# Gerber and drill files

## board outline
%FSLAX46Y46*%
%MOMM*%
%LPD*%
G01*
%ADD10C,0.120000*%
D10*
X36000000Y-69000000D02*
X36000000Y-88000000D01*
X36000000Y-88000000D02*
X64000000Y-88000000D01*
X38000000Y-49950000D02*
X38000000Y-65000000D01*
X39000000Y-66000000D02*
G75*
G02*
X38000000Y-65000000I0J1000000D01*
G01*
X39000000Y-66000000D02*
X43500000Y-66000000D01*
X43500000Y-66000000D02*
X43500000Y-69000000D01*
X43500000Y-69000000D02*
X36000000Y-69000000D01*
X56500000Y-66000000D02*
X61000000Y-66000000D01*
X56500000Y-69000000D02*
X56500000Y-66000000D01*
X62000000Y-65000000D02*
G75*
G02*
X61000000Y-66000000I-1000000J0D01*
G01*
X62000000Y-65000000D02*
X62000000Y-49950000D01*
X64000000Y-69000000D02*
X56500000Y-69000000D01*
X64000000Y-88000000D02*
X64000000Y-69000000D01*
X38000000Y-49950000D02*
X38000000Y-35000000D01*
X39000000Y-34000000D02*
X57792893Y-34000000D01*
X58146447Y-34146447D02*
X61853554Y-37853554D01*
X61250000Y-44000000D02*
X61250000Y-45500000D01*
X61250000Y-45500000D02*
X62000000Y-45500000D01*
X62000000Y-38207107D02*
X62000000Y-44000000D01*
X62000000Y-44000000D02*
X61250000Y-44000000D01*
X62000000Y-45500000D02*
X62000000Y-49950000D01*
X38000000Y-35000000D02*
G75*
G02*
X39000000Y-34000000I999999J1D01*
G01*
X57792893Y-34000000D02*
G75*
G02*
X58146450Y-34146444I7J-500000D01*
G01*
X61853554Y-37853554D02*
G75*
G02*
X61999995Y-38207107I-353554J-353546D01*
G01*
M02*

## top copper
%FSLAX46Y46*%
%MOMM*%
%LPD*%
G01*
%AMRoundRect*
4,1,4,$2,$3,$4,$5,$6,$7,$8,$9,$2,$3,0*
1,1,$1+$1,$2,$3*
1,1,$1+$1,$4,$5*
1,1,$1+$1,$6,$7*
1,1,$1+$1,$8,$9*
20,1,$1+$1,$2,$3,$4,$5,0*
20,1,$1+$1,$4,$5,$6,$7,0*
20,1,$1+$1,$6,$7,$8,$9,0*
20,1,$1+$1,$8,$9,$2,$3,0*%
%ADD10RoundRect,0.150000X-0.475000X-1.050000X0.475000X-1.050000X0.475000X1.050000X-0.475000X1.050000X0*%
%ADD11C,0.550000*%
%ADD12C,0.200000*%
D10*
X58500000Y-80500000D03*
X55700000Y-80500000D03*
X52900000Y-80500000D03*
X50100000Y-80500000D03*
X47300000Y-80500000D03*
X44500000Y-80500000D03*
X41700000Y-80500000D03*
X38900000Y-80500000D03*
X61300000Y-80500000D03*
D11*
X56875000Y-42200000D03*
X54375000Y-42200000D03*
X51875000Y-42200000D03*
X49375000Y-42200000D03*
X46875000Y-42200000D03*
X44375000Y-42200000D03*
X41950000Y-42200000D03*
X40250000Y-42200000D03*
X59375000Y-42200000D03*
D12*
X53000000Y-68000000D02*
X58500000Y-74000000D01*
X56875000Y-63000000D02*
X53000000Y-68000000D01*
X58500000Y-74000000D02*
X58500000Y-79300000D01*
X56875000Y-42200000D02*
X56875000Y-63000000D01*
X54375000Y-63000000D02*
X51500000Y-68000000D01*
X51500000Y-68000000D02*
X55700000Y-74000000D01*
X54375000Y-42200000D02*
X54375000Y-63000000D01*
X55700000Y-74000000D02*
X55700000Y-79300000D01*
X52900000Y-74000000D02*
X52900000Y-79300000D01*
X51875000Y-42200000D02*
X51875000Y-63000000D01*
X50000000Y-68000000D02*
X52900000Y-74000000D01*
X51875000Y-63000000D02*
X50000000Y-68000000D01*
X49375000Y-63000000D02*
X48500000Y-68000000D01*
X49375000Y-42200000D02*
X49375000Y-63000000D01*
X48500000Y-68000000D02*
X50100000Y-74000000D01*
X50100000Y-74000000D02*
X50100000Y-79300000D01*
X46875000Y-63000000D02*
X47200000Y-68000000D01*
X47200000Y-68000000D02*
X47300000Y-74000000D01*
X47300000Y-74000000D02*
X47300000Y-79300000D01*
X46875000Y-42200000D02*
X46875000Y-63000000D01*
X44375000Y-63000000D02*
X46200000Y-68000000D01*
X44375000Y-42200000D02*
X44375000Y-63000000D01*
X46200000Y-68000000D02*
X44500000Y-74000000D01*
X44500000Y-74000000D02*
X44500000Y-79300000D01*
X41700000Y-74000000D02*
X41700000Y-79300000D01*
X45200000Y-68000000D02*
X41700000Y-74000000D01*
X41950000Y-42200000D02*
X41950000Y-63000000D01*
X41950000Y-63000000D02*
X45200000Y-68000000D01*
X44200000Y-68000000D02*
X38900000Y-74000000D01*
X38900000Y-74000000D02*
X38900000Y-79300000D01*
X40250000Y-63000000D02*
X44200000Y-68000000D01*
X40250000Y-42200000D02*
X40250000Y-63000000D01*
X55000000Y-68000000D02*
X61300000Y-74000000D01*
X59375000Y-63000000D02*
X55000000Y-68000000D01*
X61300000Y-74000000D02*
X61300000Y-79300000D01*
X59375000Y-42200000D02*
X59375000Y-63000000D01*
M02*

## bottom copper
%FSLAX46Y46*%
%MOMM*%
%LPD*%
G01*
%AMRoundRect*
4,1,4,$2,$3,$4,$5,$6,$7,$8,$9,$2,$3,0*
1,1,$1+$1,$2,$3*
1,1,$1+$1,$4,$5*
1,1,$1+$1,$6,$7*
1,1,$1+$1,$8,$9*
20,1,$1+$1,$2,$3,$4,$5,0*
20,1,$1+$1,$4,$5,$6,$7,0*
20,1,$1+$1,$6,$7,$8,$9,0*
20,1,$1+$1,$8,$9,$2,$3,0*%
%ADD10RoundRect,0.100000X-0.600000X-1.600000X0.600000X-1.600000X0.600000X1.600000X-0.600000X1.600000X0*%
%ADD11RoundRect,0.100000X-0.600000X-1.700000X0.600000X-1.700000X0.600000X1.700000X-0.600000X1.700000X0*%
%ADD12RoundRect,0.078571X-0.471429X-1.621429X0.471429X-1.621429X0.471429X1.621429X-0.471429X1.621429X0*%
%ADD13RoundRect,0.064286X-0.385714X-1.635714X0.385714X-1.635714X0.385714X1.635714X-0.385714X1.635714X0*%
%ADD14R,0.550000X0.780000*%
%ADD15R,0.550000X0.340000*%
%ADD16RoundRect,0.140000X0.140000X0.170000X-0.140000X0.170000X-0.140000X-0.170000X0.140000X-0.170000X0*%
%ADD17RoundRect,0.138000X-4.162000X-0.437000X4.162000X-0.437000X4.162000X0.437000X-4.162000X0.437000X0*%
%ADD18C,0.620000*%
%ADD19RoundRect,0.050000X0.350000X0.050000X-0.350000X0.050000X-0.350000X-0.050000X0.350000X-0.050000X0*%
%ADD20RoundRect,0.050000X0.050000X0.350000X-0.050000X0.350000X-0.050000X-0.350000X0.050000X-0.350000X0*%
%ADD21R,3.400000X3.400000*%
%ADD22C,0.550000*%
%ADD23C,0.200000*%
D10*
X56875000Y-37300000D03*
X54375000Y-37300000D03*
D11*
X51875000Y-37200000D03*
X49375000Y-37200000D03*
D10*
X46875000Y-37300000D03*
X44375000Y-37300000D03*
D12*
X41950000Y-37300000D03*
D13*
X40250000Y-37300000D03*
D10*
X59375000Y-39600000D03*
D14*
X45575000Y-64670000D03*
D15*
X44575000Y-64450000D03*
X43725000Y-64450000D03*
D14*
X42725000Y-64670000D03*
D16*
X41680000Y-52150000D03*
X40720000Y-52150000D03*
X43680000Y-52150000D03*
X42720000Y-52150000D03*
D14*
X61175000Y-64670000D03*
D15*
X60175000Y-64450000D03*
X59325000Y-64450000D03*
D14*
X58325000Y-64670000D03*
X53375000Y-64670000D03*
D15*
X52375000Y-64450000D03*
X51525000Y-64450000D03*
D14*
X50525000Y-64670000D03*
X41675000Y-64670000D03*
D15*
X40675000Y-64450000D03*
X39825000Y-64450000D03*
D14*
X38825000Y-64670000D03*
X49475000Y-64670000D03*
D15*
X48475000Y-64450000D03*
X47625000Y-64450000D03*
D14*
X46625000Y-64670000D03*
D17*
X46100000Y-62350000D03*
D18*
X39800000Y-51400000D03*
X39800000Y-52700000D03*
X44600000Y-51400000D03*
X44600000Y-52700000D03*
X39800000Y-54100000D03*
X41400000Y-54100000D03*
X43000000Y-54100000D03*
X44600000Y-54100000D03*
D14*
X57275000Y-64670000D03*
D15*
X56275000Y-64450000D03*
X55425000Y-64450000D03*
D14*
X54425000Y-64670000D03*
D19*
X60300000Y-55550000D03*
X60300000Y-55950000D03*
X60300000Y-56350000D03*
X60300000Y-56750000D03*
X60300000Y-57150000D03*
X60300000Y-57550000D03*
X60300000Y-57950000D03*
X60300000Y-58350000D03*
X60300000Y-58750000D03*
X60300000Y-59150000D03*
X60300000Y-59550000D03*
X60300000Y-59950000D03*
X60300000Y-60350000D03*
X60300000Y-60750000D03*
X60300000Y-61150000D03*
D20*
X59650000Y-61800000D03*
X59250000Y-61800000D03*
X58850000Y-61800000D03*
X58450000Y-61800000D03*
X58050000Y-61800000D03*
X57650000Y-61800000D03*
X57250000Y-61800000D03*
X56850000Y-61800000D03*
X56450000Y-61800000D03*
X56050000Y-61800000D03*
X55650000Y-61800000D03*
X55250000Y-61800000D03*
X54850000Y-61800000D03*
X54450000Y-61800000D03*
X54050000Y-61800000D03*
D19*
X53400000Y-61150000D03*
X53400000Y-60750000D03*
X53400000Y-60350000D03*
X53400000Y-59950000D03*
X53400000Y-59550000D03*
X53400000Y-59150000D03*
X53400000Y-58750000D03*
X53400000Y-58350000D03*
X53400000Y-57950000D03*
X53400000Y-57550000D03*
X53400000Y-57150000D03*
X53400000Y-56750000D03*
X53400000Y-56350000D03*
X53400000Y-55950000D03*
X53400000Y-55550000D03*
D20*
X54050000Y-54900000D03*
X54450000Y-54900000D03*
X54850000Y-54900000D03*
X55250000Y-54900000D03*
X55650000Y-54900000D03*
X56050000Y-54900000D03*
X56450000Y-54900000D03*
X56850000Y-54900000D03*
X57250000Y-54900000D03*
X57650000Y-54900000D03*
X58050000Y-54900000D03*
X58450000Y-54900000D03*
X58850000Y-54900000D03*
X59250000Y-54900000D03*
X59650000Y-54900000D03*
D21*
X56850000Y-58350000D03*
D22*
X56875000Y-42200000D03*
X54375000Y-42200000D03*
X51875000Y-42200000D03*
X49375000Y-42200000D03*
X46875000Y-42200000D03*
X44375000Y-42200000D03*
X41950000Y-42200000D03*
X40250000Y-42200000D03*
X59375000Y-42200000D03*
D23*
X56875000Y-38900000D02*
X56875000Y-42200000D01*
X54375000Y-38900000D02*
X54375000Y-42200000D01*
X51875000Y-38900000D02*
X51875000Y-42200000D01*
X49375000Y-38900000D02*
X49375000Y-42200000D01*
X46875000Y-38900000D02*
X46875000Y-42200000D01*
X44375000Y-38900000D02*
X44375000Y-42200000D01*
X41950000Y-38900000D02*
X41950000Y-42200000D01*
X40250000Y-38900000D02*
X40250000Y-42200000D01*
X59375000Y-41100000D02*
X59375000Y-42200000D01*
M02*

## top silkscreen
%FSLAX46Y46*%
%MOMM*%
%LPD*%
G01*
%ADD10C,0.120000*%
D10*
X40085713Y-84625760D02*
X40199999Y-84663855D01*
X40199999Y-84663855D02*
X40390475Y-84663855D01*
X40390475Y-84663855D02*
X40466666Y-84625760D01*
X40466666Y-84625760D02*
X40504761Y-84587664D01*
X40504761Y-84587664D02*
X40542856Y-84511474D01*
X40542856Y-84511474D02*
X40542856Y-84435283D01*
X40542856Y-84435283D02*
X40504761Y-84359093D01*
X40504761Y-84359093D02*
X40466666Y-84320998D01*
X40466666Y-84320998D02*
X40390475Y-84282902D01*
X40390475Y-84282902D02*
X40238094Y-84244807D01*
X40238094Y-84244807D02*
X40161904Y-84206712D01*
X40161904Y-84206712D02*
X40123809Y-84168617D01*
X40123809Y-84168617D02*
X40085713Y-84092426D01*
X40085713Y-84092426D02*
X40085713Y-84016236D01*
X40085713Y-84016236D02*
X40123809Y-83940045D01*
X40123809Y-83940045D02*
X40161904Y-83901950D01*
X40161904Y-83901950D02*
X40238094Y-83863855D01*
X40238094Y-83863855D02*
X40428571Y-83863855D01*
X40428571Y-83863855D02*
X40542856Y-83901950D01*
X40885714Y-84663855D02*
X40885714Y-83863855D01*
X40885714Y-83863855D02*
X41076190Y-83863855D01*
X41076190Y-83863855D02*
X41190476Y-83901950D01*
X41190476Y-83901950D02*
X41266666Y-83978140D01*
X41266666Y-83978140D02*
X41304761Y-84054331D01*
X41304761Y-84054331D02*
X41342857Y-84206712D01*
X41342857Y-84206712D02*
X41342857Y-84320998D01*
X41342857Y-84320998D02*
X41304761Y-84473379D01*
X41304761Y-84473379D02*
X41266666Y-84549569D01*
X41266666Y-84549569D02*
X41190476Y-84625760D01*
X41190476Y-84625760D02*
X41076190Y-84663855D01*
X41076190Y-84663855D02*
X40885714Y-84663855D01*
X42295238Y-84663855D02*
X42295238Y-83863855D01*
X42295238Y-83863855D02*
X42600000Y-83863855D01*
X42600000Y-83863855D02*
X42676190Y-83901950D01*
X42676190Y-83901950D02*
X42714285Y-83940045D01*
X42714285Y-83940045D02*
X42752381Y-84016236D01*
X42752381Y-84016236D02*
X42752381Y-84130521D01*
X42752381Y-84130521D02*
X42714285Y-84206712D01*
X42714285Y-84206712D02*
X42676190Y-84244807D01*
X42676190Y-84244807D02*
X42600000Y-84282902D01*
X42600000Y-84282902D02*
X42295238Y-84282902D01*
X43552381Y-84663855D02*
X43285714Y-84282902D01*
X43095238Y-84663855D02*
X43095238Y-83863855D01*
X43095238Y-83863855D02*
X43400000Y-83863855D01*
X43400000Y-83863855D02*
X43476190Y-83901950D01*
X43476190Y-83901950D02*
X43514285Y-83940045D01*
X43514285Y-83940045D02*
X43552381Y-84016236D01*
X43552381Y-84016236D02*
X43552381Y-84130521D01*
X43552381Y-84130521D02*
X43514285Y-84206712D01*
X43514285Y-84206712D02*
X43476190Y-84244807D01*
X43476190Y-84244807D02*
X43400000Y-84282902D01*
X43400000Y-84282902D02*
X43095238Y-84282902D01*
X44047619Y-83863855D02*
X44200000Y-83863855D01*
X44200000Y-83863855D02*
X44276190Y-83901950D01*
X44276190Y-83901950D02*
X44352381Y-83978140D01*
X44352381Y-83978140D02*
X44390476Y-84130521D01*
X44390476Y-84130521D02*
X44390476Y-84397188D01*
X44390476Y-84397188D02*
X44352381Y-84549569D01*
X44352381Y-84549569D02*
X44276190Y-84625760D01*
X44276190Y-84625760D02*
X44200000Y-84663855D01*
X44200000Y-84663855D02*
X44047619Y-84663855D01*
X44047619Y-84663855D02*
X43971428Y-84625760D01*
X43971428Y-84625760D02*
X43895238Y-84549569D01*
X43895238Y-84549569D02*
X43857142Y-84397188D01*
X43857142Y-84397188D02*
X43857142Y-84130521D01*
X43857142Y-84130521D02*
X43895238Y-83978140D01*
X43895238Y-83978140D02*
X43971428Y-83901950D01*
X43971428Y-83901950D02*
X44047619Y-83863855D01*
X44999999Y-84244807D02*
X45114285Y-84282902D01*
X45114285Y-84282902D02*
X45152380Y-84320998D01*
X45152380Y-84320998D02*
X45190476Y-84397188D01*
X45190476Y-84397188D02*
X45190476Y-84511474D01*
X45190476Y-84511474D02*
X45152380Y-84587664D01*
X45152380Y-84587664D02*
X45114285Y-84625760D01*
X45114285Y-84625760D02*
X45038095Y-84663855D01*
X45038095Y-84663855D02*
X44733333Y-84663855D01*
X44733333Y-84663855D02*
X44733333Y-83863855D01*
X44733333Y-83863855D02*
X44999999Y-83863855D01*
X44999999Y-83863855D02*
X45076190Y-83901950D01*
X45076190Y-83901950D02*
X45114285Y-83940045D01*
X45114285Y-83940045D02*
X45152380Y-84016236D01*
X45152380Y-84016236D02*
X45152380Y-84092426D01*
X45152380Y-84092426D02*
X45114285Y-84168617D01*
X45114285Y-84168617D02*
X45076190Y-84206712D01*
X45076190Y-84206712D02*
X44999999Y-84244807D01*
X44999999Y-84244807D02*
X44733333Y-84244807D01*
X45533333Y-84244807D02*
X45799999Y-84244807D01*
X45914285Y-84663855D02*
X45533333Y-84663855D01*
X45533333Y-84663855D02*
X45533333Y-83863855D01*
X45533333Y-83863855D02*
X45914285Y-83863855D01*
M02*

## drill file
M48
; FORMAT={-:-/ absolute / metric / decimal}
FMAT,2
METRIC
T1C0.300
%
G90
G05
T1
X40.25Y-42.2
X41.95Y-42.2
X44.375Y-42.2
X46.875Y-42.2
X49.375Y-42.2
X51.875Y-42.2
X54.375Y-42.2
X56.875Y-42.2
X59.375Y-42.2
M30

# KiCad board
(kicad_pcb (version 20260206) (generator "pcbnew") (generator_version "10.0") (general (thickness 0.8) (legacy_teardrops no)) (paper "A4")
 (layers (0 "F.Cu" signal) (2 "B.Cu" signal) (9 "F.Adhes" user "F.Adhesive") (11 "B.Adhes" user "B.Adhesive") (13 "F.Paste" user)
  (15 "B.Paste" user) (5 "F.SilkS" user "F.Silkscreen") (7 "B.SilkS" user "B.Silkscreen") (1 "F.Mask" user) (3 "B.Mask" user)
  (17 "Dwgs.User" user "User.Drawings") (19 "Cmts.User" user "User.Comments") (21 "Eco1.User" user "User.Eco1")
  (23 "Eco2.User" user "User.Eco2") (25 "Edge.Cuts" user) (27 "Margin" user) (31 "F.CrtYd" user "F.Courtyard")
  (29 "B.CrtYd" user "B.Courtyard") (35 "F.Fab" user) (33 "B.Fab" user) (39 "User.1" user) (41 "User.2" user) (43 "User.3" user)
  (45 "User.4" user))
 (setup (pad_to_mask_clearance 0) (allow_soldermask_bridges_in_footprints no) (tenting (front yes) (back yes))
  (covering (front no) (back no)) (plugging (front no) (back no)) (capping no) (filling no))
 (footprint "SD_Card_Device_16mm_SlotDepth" (layer "F.Cu") (at 50 50)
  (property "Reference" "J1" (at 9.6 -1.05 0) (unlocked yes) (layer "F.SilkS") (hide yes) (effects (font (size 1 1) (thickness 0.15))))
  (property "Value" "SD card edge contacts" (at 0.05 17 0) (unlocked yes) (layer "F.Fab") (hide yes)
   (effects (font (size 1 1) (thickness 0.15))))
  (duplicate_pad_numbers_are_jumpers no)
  (fp_line (start -12 -0.05) (end -12 -15) (stroke (width 0.12) (type default)) (layer "Edge.Cuts"))
  (fp_line (start -11 -16) (end 7.792893 -16) (stroke (width 0.12) (type default)) (layer "Edge.Cuts"))
  (fp_line (start 8.146447 -15.853553) (end 11.853554 -12.146446) (stroke (width 0.12) (type default)) (layer "Edge.Cuts"))
  (fp_line (start 11.25 -6) (end 11.25 -4.5) (stroke (width 0.12) (type default)) (layer "Edge.Cuts"))
  (fp_line (start 11.25 -4.5) (end 12 -4.5) (stroke (width 0.12) (type default)) (layer "Edge.Cuts"))
  (fp_line (start 12 -11.792893) (end 12 -6) (stroke (width 0.12) (type default)) (layer "Edge.Cuts"))
  (fp_line (start 12 -6) (end 11.25 -6) (stroke (width 0.12) (type default)) (layer "Edge.Cuts"))
  (fp_line (start 12 -4.5) (end 12 -0.05) (stroke (width 0.12) (type default)) (layer "Edge.Cuts"))
  (fp_arc (start -12 -15) (mid -11.707107 -15.707107) (end -11 -16) (stroke (width 0.12) (type default)) (layer "Edge.Cuts"))
  (fp_arc (start 7.792893 -16) (mid 7.984235 -15.96194) (end 8.146447 -15.853553) (stroke (width 0.12) (type default)) (layer "Edge.Cuts"))
  (fp_arc (start 11.853554 -12.146446) (mid 11.96194 -11.984234) (end 12 -11.792893) (stroke (width 0.12) (type default))
   (layer "Edge.Cuts"))
  (pad "1" connect roundrect (at 6.875 -12.7) (size 1.4 3.4) (layers "B.Cu" "B.Mask") (roundrect_rratio 0.07142857143) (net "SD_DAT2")
   (clearance 0.05))
  (pad "2" connect roundrect (at 4.375 -12.7) (size 1.4 3.4) (layers "B.Cu" "B.Mask") (roundrect_rratio 0.07142857143) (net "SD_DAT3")
   (clearance 0.05))
  (pad "3" connect roundrect (at 1.875 -12.8) (size 1.4 3.6) (layers "B.Cu" "B.Mask") (roundrect_rratio 0.07142857143) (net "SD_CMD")
   (clearance 0.05))
  (pad "4" connect roundrect (at -0.625 -12.8) (size 1.4 3.6) (layers "B.Cu" "B.Mask") (roundrect_rratio 0.07142857143) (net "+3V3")
   (clearance 0.05))
  (pad "5" connect roundrect (at -3.125 -12.7) (size 1.4 3.4) (layers "B.Cu" "B.Mask") (roundrect_rratio 0.07142857143) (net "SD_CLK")
   (clearance 0.05))
  (pad "6" connect roundrect (at -5.625 -12.7) (size 1.4 3.4) (layers "B.Cu" "B.Mask") (roundrect_rratio 0.07142857143) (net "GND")
   (clearance 0.05))
  (pad "7" connect roundrect (at -8.05 -12.7) (size 1.1 3.4) (layers "B.Cu" "B.Mask") (roundrect_rratio 0.07142857143) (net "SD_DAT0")
   (clearance 0.05))
  (pad "8" connect roundrect (at -9.75 -12.7) (size 0.9 3.4) (layers "B.Cu" "B.Mask") (roundrect_rratio 0.07142857143) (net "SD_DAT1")
   (clearance 0.05))
  (pad "9" connect roundrect (at 9.375 -10.4) (size 1.4 3.4) (layers "B.Cu" "B.Mask") (roundrect_rratio 0.07142857143) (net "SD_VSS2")
   (clearance 0.05))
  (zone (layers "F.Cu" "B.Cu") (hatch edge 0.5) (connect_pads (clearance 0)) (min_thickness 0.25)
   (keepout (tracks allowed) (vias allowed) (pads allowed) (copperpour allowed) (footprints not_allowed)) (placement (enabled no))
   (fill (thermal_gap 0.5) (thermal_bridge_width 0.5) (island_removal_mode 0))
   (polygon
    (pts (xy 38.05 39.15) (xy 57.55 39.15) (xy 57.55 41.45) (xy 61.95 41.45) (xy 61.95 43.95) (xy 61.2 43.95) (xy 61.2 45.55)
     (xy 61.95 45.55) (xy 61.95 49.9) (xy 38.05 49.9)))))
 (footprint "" (layer "F.Cu") (at 0 0)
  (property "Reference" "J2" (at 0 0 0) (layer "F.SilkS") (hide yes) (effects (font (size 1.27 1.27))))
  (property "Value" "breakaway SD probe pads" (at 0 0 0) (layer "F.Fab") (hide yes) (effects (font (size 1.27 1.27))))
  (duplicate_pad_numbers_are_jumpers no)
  (pad "1" smd roundrect (at 58.5 80.5) (size 1.25 2.4) (layers "F.Cu" "F.Mask" "F.Paste") (roundrect_rratio 0.12) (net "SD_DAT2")
   (thermal_bridge_angle 45))
  (pad "2" smd roundrect (at 55.7 80.5) (size 1.25 2.4) (layers "F.Cu" "F.Mask" "F.Paste") (roundrect_rratio 0.12) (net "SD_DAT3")
   (thermal_bridge_angle 45))
  (pad "3" smd roundrect (at 52.9 80.5) (size 1.25 2.4) (layers "F.Cu" "F.Mask" "F.Paste") (roundrect_rratio 0.12) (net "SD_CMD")
   (thermal_bridge_angle 45))
  (pad "4" smd roundrect (at 50.1 80.5) (size 1.25 2.4) (layers "F.Cu" "F.Mask" "F.Paste") (roundrect_rratio 0.12) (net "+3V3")
   (thermal_bridge_angle 45))
  (pad "5" smd roundrect (at 47.3 80.5) (size 1.25 2.4) (layers "F.Cu" "F.Mask" "F.Paste") (roundrect_rratio 0.12) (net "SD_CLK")
   (thermal_bridge_angle 45))
  (pad "6" smd roundrect (at 44.5 80.5) (size 1.25 2.4) (layers "F.Cu" "F.Mask" "F.Paste") (roundrect_rratio 0.12) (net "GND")
   (thermal_bridge_angle 45))
  (pad "7" smd roundrect (at 41.7 80.5) (size 1.25 2.4) (layers "F.Cu" "F.Mask" "F.Paste") (roundrect_rratio 0.12) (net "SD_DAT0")
   (thermal_bridge_angle 45))
  (pad "8" smd roundrect (at 38.9 80.5) (size 1.25 2.4) (layers "F.Cu" "F.Mask" "F.Paste") (roundrect_rratio 0.12) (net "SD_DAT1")
   (thermal_bridge_angle 45))
  (pad "9" smd roundrect (at 61.3 80.5) (size 1.25 2.4) (layers "F.Cu" "F.Mask" "F.Paste") (roundrect_rratio 0.12) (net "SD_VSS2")
   (thermal_bridge_angle 45)))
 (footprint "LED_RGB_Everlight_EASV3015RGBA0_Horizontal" (layer "B.Cu") (at 44.15 65.2 180)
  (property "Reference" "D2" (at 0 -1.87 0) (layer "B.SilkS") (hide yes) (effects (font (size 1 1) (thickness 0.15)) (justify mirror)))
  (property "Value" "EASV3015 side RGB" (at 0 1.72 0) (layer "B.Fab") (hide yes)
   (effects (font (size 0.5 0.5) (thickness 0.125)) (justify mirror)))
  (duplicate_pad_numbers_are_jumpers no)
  (pad "1" smd rect (at -1.425 0.53 180) (size 0.55 0.78) (layers "B.Cu" "B.Mask" "B.Paste"))
  (pad "2" smd rect (at -0.425 0.75 180) (size 0.55 0.34) (layers "B.Cu" "B.Mask" "B.Paste"))
  (pad "3" smd rect (at 0.425 0.75 180) (size 0.55 0.34) (layers "B.Cu" "B.Mask" "B.Paste"))
  (pad "4" smd rect (at 1.425 0.53 180) (size 0.55 0.78) (layers "B.Cu" "B.Mask" "B.Paste")))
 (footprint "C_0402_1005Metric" (layer "B.Cu") (at 41.2 52.15 180)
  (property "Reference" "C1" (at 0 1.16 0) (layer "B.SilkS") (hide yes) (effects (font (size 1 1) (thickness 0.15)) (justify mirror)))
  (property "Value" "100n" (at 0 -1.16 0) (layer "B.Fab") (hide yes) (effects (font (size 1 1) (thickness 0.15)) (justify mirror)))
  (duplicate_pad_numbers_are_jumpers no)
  (pad "1" smd roundrect (at -0.48 0 180) (size 0.56 0.62) (layers "B.Cu" "B.Mask" "B.Paste") (roundrect_rratio 0.25))
  (pad "2" smd roundrect (at 0.48 0 180) (size 0.56 0.62) (layers "B.Cu" "B.Mask" "B.Paste") (roundrect_rratio 0.25)))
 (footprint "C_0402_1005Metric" (layer "B.Cu") (at 43.2 52.15 180)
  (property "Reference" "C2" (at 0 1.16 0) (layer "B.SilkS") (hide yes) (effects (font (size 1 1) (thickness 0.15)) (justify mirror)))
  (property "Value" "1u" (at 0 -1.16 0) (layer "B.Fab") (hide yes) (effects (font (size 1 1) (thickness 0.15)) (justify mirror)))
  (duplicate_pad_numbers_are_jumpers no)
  (pad "1" smd roundrect (at -0.48 0 180) (size 0.56 0.62) (layers "B.Cu" "B.Mask" "B.Paste") (roundrect_rratio 0.25))
  (pad "2" smd roundrect (at 0.48 0 180) (size 0.56 0.62) (layers "B.Cu" "B.Mask" "B.Paste") (roundrect_rratio 0.25)))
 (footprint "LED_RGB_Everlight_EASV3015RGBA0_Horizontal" (layer "B.Cu") (at 59.75 65.2 180)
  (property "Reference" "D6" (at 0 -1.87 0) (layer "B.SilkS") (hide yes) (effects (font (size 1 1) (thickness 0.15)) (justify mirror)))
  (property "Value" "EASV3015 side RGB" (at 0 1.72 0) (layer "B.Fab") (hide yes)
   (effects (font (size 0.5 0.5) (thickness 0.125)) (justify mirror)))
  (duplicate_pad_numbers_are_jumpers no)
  (pad "1" smd rect (at -1.425 0.53 180) (size 0.55 0.78) (layers "B.Cu" "B.Mask" "B.Paste"))
  (pad "2" smd rect (at -0.425 0.75 180) (size 0.55 0.34) (layers "B.Cu" "B.Mask" "B.Paste"))
  (pad "3" smd rect (at 0.425 0.75 180) (size 0.55 0.34) (layers "B.Cu" "B.Mask" "B.Paste"))
  (pad "4" smd rect (at 1.425 0.53 180) (size 0.55 0.78) (layers "B.Cu" "B.Mask" "B.Paste")))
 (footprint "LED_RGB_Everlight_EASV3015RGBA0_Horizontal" (layer "B.Cu") (at 51.95 65.2 180)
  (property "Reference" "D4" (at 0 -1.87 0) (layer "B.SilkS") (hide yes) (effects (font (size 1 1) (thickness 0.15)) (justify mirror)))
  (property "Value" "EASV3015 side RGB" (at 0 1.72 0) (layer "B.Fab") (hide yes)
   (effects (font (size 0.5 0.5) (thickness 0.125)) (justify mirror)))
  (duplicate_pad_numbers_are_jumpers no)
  (pad "1" smd rect (at -1.425 0.53 180) (size 0.55 0.78) (layers "B.Cu" "B.Mask" "B.Paste"))
  (pad "2" smd rect (at -0.425 0.75 180) (size 0.55 0.34) (layers "B.Cu" "B.Mask" "B.Paste"))
  (pad "3" smd rect (at 0.425 0.75 180) (size 0.55 0.34) (layers "B.Cu" "B.Mask" "B.Paste"))
  (pad "4" smd rect (at 1.425 0.53 180) (size 0.55 0.78) (layers "B.Cu" "B.Mask" "B.Paste")))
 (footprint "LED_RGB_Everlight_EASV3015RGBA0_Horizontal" (layer "B.Cu") (at 40.25 65.2 180)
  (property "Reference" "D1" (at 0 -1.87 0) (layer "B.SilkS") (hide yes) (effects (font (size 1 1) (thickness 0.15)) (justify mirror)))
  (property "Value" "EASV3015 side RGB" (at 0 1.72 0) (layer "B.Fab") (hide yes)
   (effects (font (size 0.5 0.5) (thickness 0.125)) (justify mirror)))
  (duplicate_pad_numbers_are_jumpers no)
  (pad "1" smd rect (at -1.425 0.53 180) (size 0.55 0.78) (layers "B.Cu" "B.Mask" "B.Paste"))
  (pad "2" smd rect (at -0.425 0.75 180) (size 0.55 0.34) (layers "B.Cu" "B.Mask" "B.Paste"))
  (pad "3" smd rect (at 0.425 0.75 180) (size 0.55 0.34) (layers "B.Cu" "B.Mask" "B.Paste"))
  (pad "4" smd rect (at 1.425 0.53 180) (size 0.55 0.78) (layers "B.Cu" "B.Mask" "B.Paste")))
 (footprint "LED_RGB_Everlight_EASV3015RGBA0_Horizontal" (layer "B.Cu") (at 48.05 65.2 180)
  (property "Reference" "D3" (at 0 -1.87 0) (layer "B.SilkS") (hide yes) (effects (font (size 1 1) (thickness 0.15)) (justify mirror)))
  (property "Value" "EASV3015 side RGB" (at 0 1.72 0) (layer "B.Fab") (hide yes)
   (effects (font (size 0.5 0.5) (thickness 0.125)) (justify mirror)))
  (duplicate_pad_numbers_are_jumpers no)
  (pad "1" smd rect (at -1.425 0.53 180) (size 0.55 0.78) (layers "B.Cu" "B.Mask" "B.Paste"))
  (pad "2" smd rect (at -0.425 0.75 180) (size 0.55 0.34) (layers "B.Cu" "B.Mask" "B.Paste"))
  (pad "3" smd rect (at 0.425 0.75 180) (size 0.55 0.34) (layers "B.Cu" "B.Mask" "B.Paste"))
  (pad "4" smd rect (at 1.425 0.53 180) (size 0.55 0.78) (layers "B.Cu" "B.Mask" "B.Paste")))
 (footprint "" (layer "B.Cu") (at 0 0)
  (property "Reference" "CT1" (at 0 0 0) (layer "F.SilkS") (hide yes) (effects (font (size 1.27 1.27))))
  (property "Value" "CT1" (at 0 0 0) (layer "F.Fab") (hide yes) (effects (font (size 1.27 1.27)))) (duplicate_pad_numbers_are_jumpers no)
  (pad "1" smd roundrect (at 46.1 62.35) (size 8.6 1.15) (layers "B.Cu" "B.Mask" "B.Paste") (roundrect_rratio 0.12)
   (thermal_bridge_angle 45)))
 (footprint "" (layer "B.Cu") (at 0 0)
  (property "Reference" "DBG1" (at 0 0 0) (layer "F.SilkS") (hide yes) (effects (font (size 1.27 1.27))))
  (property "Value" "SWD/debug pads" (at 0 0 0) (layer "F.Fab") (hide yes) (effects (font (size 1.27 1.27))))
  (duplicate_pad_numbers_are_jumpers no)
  (pad "1" smd circle (at 39.8 51.4) (size 0.62 0.62) (layers "B.Cu" "B.Mask" "B.Paste"))
  (pad "2" smd circle (at 39.8 52.7) (size 0.62 0.62) (layers "B.Cu" "B.Mask" "B.Paste"))
  (pad "3" smd circle (at 44.6 51.4) (size 0.62 0.62) (layers "B.Cu" "B.Mask" "B.Paste"))
  (pad "4" smd circle (at 44.6 52.7) (size 0.62 0.62) (layers "B.Cu" "B.Mask" "B.Paste"))
  (pad "5" smd circle (at 39.8 54.1) (size 0.62 0.62) (layers "B.Cu" "B.Mask" "B.Paste"))
  (pad "6" smd circle (at 41.4 54.1) (size 0.62 0.62) (layers "B.Cu" "B.Mask" "B.Paste"))
  (pad "7" smd circle (at 43 54.1) (size 0.62 0.62) (layers "B.Cu" "B.Mask" "B.Paste"))
  (pad "8" smd circle (at 44.6 54.1) (size 0.62 0.62) (layers "B.Cu" "B.Mask" "B.Paste")))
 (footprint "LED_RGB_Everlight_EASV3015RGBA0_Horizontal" (layer "B.Cu") (at 55.85 65.2 180)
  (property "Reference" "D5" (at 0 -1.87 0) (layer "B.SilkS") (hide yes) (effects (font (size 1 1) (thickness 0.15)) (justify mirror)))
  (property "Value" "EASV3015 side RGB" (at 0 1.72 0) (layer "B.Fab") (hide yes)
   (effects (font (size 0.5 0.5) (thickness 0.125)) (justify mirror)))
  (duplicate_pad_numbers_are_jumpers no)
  (pad "1" smd rect (at -1.425 0.53 180) (size 0.55 0.78) (layers "B.Cu" "B.Mask" "B.Paste"))
  (pad "2" smd rect (at -0.425 0.75 180) (size 0.55 0.34) (layers "B.Cu" "B.Mask" "B.Paste"))
  (pad "3" smd rect (at 0.425 0.75 180) (size 0.55 0.34) (layers "B.Cu" "B.Mask" "B.Paste"))
  (pad "4" smd rect (at 1.425 0.53 180) (size 0.55 0.78) (layers "B.Cu" "B.Mask" "B.Paste")))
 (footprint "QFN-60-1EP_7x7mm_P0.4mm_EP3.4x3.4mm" (layer "B.Cu") (at 56.85 58.35 180)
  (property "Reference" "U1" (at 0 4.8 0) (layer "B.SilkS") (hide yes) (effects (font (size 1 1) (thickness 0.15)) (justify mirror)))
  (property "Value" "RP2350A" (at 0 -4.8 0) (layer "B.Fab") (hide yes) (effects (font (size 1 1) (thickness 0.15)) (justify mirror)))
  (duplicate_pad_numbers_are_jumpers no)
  (pad "" smd roundrect (at -1.13 -1.13 180) (size 0.91 0.91) (layers "B.Paste") (roundrect_rratio 0.25))
  (pad "" smd roundrect (at -1.13 0 180) (size 0.91 0.91) (layers "B.Paste") (roundrect_rratio 0.25))
  (pad "" smd roundrect (at -1.13 1.13 180) (size 0.91 0.91) (layers "B.Paste") (roundrect_rratio 0.25))
  (pad "" smd roundrect (at 0 -1.13 180) (size 0.91 0.91) (layers "B.Paste") (roundrect_rratio 0.25))
  (pad "" smd roundrect (at 0 0 180) (size 0.91 0.91) (layers "B.Paste") (roundrect_rratio 0.25))
  (pad "" smd roundrect (at 0 1.13 180) (size 0.91 0.91) (layers "B.Paste") (roundrect_rratio 0.25))
  (pad "" smd roundrect (at 1.13 -1.13 180) (size 0.91 0.91) (layers "B.Paste") (roundrect_rratio 0.25))
  (pad "" smd roundrect (at 1.13 0 180) (size 0.91 0.91) (layers "B.Paste") (roundrect_rratio 0.25))
  (pad "" smd roundrect (at 1.13 1.13 180) (size 0.91 0.91) (layers "B.Paste") (roundrect_rratio 0.25))
  (pad "1" smd roundrect (at -3.45 2.8 180) (size 0.8 0.2) (layers "B.Cu" "B.Mask" "B.Paste") (roundrect_rratio 0.25))
  (pad "2" smd roundrect (at -3.45 2.4 180) (size 0.8 0.2) (layers "B.Cu" "B.Mask" "B.Paste") (roundrect_rratio 0.25))
  (pad "3" smd roundrect (at -3.45 2 180) (size 0.8 0.2) (layers "B.Cu" "B.Mask" "B.Paste") (roundrect_rratio 0.25))
  (pad "4" smd roundrect (at -3.45 1.6 180) (size 0.8 0.2) (layers "B.Cu" "B.Mask" "B.Paste") (roundrect_rratio 0.25))
  (pad "5" smd roundrect (at -3.45 1.2 180) (size 0.8 0.2) (layers "B.Cu" "B.Mask" "B.Paste") (roundrect_rratio 0.25))
  (pad "6" smd roundrect (at -3.45 0.8 180) (size 0.8 0.2) (layers "B.Cu" "B.Mask" "B.Paste") (roundrect_rratio 0.25))
  (pad "7" smd roundrect (at -3.45 0.4 180) (size 0.8 0.2) (layers "B.Cu" "B.Mask" "B.Paste") (roundrect_rratio 0.25))
  (pad "8" smd roundrect (at -3.45 0 180) (size 0.8 0.2) (layers "B.Cu" "B.Mask" "B.Paste") (roundrect_rratio 0.25))
  (pad "9" smd roundrect (at -3.45 -0.4 180) (size 0.8 0.2) (layers "B.Cu" "B.Mask" "B.Paste") (roundrect_rratio 0.25))
  (pad "10" smd roundrect (at -3.45 -0.8 180) (size 0.8 0.2) (layers "B.Cu" "B.Mask" "B.Paste") (roundrect_rratio 0.25))
  (pad "11" smd roundrect (at -3.45 -1.2 180) (size 0.8 0.2) (layers "B.Cu" "B.Mask" "B.Paste") (roundrect_rratio 0.25))
  (pad "12" smd roundrect (at -3.45 -1.6 180) (size 0.8 0.2) (layers "B.Cu" "B.Mask" "B.Paste") (roundrect_rratio 0.25))
  (pad "13" smd roundrect (at -3.45 -2 180) (size 0.8 0.2) (layers "B.Cu" "B.Mask" "B.Paste") (roundrect_rratio 0.25))
  (pad "14" smd roundrect (at -3.45 -2.4 180) (size 0.8 0.2) (layers "B.Cu" "B.Mask" "B.Paste") (roundrect_rratio 0.25))
  (pad "15" smd roundrect (at -3.45 -2.8 180) (size 0.8 0.2) (layers "B.Cu" "B.Mask" "B.Paste") (roundrect_rratio 0.25))
  (pad "16" smd roundrect (at -2.8 -3.45 180) (size 0.2 0.8) (layers "B.Cu" "B.Mask" "B.Paste") (roundrect_rratio 0.25))
  (pad "17" smd roundrect (at -2.4 -3.45 180) (size 0.2 0.8) (layers "B.Cu" "B.Mask" "B.Paste") (roundrect_rratio 0.25))
  (pad "18" smd roundrect (at -2 -3.45 180) (size 0.2 0.8) (layers "B.Cu" "B.Mask" "B.Paste") (roundrect_rratio 0.25))
  (pad "19" smd roundrect (at -1.6 -3.45 180) (size 0.2 0.8) (layers "B.Cu" "B.Mask" "B.Paste") (roundrect_rratio 0.25))
  (pad "20" smd roundrect (at -1.2 -3.45 180) (size 0.2 0.8) (layers "B.Cu" "B.Mask" "B.Paste") (roundrect_rratio 0.25))
  (pad "21" smd roundrect (at -0.8 -3.45 180) (size 0.2 0.8) (layers "B.Cu" "B.Mask" "B.Paste") (roundrect_rratio 0.25))
  (pad "22" smd roundrect (at -0.4 -3.45 180) (size 0.2 0.8) (layers "B.Cu" "B.Mask" "B.Paste") (roundrect_rratio 0.25))
  (pad "23" smd roundrect (at 0 -3.45 180) (size 0.2 0.8) (layers "B.Cu" "B.Mask" "B.Paste") (roundrect_rratio 0.25))
  (pad "24" smd roundrect (at 0.4 -3.45 180) (size 0.2 0.8) (layers "B.Cu" "B.Mask" "B.Paste") (roundrect_rratio 0.25))
  (pad "25" smd roundrect (at 0.8 -3.45 180) (size 0.2 0.8) (layers "B.Cu" "B.Mask" "B.Paste") (roundrect_rratio 0.25))
  (pad "26" smd roundrect (at 1.2 -3.45 180) (size 0.2 0.8) (layers "B.Cu" "B.Mask" "B.Paste") (roundrect_rratio 0.25))
  (pad "27" smd roundrect (at 1.6 -3.45 180) (size 0.2 0.8) (layers "B.Cu" "B.Mask" "B.Paste") (roundrect_rratio 0.25))
  (pad "28" smd roundrect (at 2 -3.45 180) (size 0.2 0.8) (layers "B.Cu" "B.Mask" "B.Paste") (roundrect_rratio 0.25))
  (pad "29" smd roundrect (at 2.4 -3.45 180) (size 0.2 0.8) (layers "B.Cu" "B.Mask" "B.Paste") (roundrect_rratio 0.25))
  (pad "30" smd roundrect (at 2.8 -3.45 180) (size 0.2 0.8) (layers "B.Cu" "B.Mask" "B.Paste") (roundrect_rratio 0.25))
  (pad "31" smd roundrect (at 3.45 -2.8 180) (size 0.8 0.2) (layers "B.Cu" "B.Mask" "B.Paste") (roundrect_rratio 0.25))
  (pad "32" smd roundrect (at 3.45 -2.4 180) (size 0.8 0.2) (layers "B.Cu" "B.Mask" "B.Paste") (roundrect_rratio 0.25))
  (pad "33" smd roundrect (at 3.45 -2 180) (size 0.8 0.2) (layers "B.Cu" "B.Mask" "B.Paste") (roundrect_rratio 0.25))
  (pad "34" smd roundrect (at 3.45 -1.6 180) (size 0.8 0.2) (layers "B.Cu" "B.Mask" "B.Paste") (roundrect_rratio 0.25))
  (pad "35" smd roundrect (at 3.45 -1.2 180) (size 0.8 0.2) (layers "B.Cu" "B.Mask" "B.Paste") (roundrect_rratio 0.25))
  (pad "36" smd roundrect (at 3.45 -0.8 180) (size 0.8 0.2) (layers "B.Cu" "B.Mask" "B.Paste") (roundrect_rratio 0.25))
  (pad "37" smd roundrect (at 3.45 -0.4 180) (size 0.8 0.2) (layers "B.Cu" "B.Mask" "B.Paste") (roundrect_rratio 0.25))
  (pad "38" smd roundrect (at 3.45 0 180) (size 0.8 0.2) (layers "B.Cu" "B.Mask" "B.Paste") (roundrect_rratio 0.25))
  (pad "39" smd roundrect (at 3.45 0.4 180) (size 0.8 0.2) (layers "B.Cu" "B.Mask" "B.Paste") (roundrect_rratio 0.25))
  (pad "40" smd roundrect (at 3.45 0.8 180) (size 0.8 0.2) (layers "B.Cu" "B.Mask" "B.Paste") (roundrect_rratio 0.25))
  (pad "41" smd roundrect (at 3.45 1.2 180) (size 0.8 0.2) (layers "B.Cu" "B.Mask" "B.Paste") (roundrect_rratio 0.25))
  (pad "42" smd roundrect (at 3.45 1.6 180) (size 0.8 0.2) (layers "B.Cu" "B.Mask" "B.Paste") (roundrect_rratio 0.25))
  (pad "43" smd roundrect (at 3.45 2 180) (size 0.8 0.2) (layers "B.Cu" "B.Mask" "B.Paste") (roundrect_rratio 0.25))
  (pad "44" smd roundrect (at 3.45 2.4 180) (size 0.8 0.2) (layers "B.Cu" "B.Mask" "B.Paste") (roundrect_rratio 0.25))
  (pad "45" smd roundrect (at 3.45 2.8 180) (size 0.8 0.2) (layers "B.Cu" "B.Mask" "B.Paste") (roundrect_rratio 0.25))
  (pad "46" smd roundrect (at 2.8 3.45 180) (size 0.2 0.8) (layers "B.Cu" "B.Mask" "B.Paste") (roundrect_rratio 0.25))
  (pad "47" smd roundrect (at 2.4 3.45 180) (size 0.2 0.8) (layers "B.Cu" "B.Mask" "B.Paste") (roundrect_rratio 0.25))
  (pad "48" smd roundrect (at 2 3.45 180) (size 0.2 0.8) (layers "B.Cu" "B.Mask" "B.Paste") (roundrect_rratio 0.25))
  (pad "49" smd roundrect (at 1.6 3.45 180) (size 0.2 0.8) (layers "B.Cu" "B.Mask" "B.Paste") (roundrect_rratio 0.25))
  (pad "50" smd roundrect (at 1.2 3.45 180) (size 0.2 0.8) (layers "B.Cu" "B.Mask" "B.Paste") (roundrect_rratio 0.25))
  (pad "51" smd roundrect (at 0.8 3.45 180) (size 0.2 0.8) (layers "B.Cu" "B.Mask" "B.Paste") (roundrect_rratio 0.25))
  (pad "52" smd roundrect (at 0.4 3.45 180) (size 0.2 0.8) (layers "B.Cu" "B.Mask" "B.Paste") (roundrect_rratio 0.25))
  (pad "53" smd roundrect (at 0 3.45 180) (size 0.2 0.8) (layers "B.Cu" "B.Mask" "B.Paste") (roundrect_rratio 0.25))
  (pad "54" smd roundrect (at -0.4 3.45 180) (size 0.2 0.8) (layers "B.Cu" "B.Mask" "B.Paste") (roundrect_rratio 0.25))
  (pad "55" smd roundrect (at -0.8 3.45 180) (size 0.2 0.8) (layers "B.Cu" "B.Mask" "B.Paste") (roundrect_rratio 0.25))
  (pad "56" smd roundrect (at -1.2 3.45 180) (size 0.2 0.8) (layers "B.Cu" "B.Mask" "B.Paste") (roundrect_rratio 0.25))
  (pad "57" smd roundrect (at -1.6 3.45 180) (size 0.2 0.8) (layers "B.Cu" "B.Mask" "B.Paste") (roundrect_rratio 0.25))
  (pad "58" smd roundrect (at -2 3.45 180) (size 0.2 0.8) (layers "B.Cu" "B.Mask" "B.Paste") (roundrect_rratio 0.25))
  (pad "59" smd roundrect (at -2.4 3.45 180) (size 0.2 0.8) (layers "B.Cu" "B.Mask" "B.Paste") (roundrect_rratio 0.25))
  (pad "60" smd roundrect (at -2.8 3.45 180) (size 0.2 0.8) (layers "B.Cu" "B.Mask" "B.Paste") (roundrect_rratio 0.25))
  (pad "61" smd rect (at 0 0 180) (size 3.4 3.4) (layers "B.Cu" "B.Mask") (zone_connect 2)))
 (gr_line (start 36 69) (end 36 88) (stroke (width 0.12) (type default)) (layer "Edge.Cuts"))
 (gr_line (start 36 88) (end 64 88) (stroke (width 0.12) (type default)) (layer "Edge.Cuts"))
 (gr_line (start 38 49.95) (end 38 65) (stroke (width 0.12) (type default)) (layer "Edge.Cuts"))
 (gr_arc (start 39 66) (mid 38.292893 65.707107) (end 38 65) (stroke (width 0.12) (type default)) (layer "Edge.Cuts"))
 (gr_line (start 39 66) (end 43.5 66) (stroke (width 0.12) (type default)) (layer "Edge.Cuts"))
 (gr_line (start 43.5 66) (end 43.5 69) (stroke (width 0.12) (type default)) (layer "Edge.Cuts"))
 (gr_line (start 43.5 69) (end 36 69) (stroke (width 0.12) (type default)) (layer "Edge.Cuts"))
 (gr_line (start 56.5 66) (end 61 66) (stroke (width 0.12) (type default)) (layer "Edge.Cuts"))
 (gr_line (start 56.5 69) (end 56.5 66) (stroke (width 0.12) (type default)) (layer "Edge.Cuts"))
 (gr_arc (start 62 65) (mid 61.707107 65.707107) (end 61 66) (stroke (width 0.12) (type default)) (layer "Edge.Cuts"))
 (gr_line (start 62 65) (end 62 49.95) (stroke (width 0.12) (type default)) (layer "Edge.Cuts"))
 (gr_line (start 64 69) (end 56.5 69) (stroke (width 0.12) (type default)) (layer "Edge.Cuts"))
 (gr_line (start 64 88) (end 64 69) (stroke (width 0.12) (type default)) (layer "Edge.Cuts"))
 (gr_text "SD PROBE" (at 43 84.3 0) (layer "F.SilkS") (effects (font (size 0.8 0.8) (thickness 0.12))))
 (segment (start 53 68) (end 58.5 74) (width 0.2) (layer "F.Cu") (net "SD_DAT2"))
 (segment (start 56.875 63) (end 53 68) (width 0.2) (layer "F.Cu") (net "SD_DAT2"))
 (segment (start 58.5 74) (end 58.5 79.3) (width 0.2) (layer "F.Cu") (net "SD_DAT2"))
 (segment (start 56.875 42.2) (end 56.875 63) (width 0.2) (layer "F.Cu") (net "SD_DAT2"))
 (via (at 56.875 42.2) (size 0.55) (drill 0.3) (layers "F.Cu" "B.Cu") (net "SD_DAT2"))
 (segment (start 56.875 38.9) (end 56.875 42.2) (width 0.2) (layer "B.Cu") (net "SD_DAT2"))
 (segment (start 54.375 63) (end 51.5 68) (width 0.2) (layer "F.Cu") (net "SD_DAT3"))
 (segment (start 51.5 68) (end 55.7 74) (width 0.2) (layer "F.Cu") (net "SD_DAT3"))
 (segment (start 54.375 42.2) (end 54.375 63) (width 0.2) (layer "F.Cu") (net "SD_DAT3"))
 (segment (start 55.7 74) (end 55.7 79.3) (width 0.2) (layer "F.Cu") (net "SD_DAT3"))
 (via (at 54.375 42.2) (size 0.55) (drill 0.3) (layers "F.Cu" "B.Cu") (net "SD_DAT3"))
 (segment (start 54.375 38.9) (end 54.375 42.2) (width 0.2) (layer "B.Cu") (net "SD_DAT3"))
 (segment (start 52.9 74) (end 52.9 79.3) (width 0.2) (layer "F.Cu") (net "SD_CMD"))
 (segment (start 51.875 42.2) (end 51.875 63) (width 0.2) (layer "F.Cu") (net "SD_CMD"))
 (segment (start 50 68) (end 52.9 74) (width 0.2) (layer "F.Cu") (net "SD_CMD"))
 (segment (start 51.875 63) (end 50 68) (width 0.2) (layer "F.Cu") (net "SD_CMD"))
 (via (at 51.875 42.2) (size 0.55) (drill 0.3) (layers "F.Cu" "B.Cu") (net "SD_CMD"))
 (segment (start 51.875 38.9) (end 51.875 42.2) (width 0.2) (layer "B.Cu") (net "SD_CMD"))
 (segment (start 49.375 63) (end 48.5 68) (width 0.2) (layer "F.Cu") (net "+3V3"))
 (segment (start 49.375 42.2) (end 49.375 63) (width 0.2) (layer "F.Cu") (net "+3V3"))
 (segment (start 48.5 68) (end 50.1 74) (width 0.2) (layer "F.Cu") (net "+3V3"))
 (segment (start 50.1 74) (end 50.1 79.3) (width 0.2) (layer "F.Cu") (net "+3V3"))
 (via (at 49.375 42.2) (size 0.55) (drill 0.3) (layers "F.Cu" "B.Cu") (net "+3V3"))
 (segment (start 49.375 38.9) (end 49.375 42.2) (width 0.2) (layer "B.Cu") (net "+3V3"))
 (segment (start 46.875 63) (end 47.2 68) (width 0.2) (layer "F.Cu") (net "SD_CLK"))
 (segment (start 47.2 68) (end 47.3 74) (width 0.2) (layer "F.Cu") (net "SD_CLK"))
 (segment (start 47.3 74) (end 47.3 79.3) (width 0.2) (layer "F.Cu") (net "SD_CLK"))
 (segment (start 46.875 42.2) (end 46.875 63) (width 0.2) (layer "F.Cu") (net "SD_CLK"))
 (via (at 46.875 42.2) (size 0.55) (drill 0.3) (layers "F.Cu" "B.Cu") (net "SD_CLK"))
 (segment (start 46.875 38.9) (end 46.875 42.2) (width 0.2) (layer "B.Cu") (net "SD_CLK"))
 (segment (start 44.375 63) (end 46.2 68) (width 0.2) (layer "F.Cu") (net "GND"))
 (segment (start 44.375 42.2) (end 44.375 63) (width 0.2) (layer "F.Cu") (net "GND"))
 (segment (start 46.2 68) (end 44.5 74) (width 0.2) (layer "F.Cu") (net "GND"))
 (segment (start 44.5 74) (end 44.5 79.3) (width 0.2) (layer "F.Cu") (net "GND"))
 (via (at 44.375 42.2) (size 0.55) (drill 0.3) (layers "F.Cu" "B.Cu") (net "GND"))
 (segment (start 44.375 38.9) (end 44.375 42.2) (width 0.2) (layer "B.Cu") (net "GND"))
 (segment (start 41.7 74) (end 41.7 79.3) (width 0.2) (layer "F.Cu") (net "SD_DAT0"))
 (segment (start 45.2 68) (end 41.7 74) (width 0.2) (layer "F.Cu") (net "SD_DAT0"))
 (segment (start 41.95 42.2) (end 41.95 63) (width 0.2) (layer "F.Cu") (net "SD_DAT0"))
 (segment (start 41.95 63) (end 45.2 68) (width 0.2) (layer "F.Cu") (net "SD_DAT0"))
 (via (at 41.95 42.2) (size 0.55) (drill 0.3) (layers "F.Cu" "B.Cu") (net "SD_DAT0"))
 (segment (start 41.95 38.9) (end 41.95 42.2) (width 0.2) (layer "B.Cu") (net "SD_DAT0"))
 (segment (start 44.2 68) (end 38.9 74) (width 0.2) (layer "F.Cu") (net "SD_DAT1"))
 (segment (start 38.9 74) (end 38.9 79.3) (width 0.2) (layer "F.Cu") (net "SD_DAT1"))
 (segment (start 40.25 63) (end 44.2 68) (width 0.2) (layer "F.Cu") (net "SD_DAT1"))
 (segment (start 40.25 42.2) (end 40.25 63) (width 0.2) (layer "F.Cu") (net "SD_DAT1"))
 (via (at 40.25 42.2) (size 0.55) (drill 0.3) (layers "F.Cu" "B.Cu") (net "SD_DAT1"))
 (segment (start 40.25 38.9) (end 40.25 42.2) (width 0.2) (layer "B.Cu") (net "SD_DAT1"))
 (segment (start 55 68) (end 61.3 74) (width 0.2) (layer "F.Cu") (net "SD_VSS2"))
 (segment (start 59.375 63) (end 55 68) (width 0.2) (layer "F.Cu") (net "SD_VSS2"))
 (segment (start 61.3 74) (end 61.3 79.3) (width 0.2) (layer "F.Cu") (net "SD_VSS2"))
 (segment (start 59.375 42.2) (end 59.375 63) (width 0.2) (layer "F.Cu") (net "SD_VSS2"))
 (via (at 59.375 42.2) (size 0.55) (drill 0.3) (layers "F.Cu" "B.Cu") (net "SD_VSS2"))
 (segment (start 59.375 41.1) (end 59.375 42.2) (width 0.2) (layer "B.Cu") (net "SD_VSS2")))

